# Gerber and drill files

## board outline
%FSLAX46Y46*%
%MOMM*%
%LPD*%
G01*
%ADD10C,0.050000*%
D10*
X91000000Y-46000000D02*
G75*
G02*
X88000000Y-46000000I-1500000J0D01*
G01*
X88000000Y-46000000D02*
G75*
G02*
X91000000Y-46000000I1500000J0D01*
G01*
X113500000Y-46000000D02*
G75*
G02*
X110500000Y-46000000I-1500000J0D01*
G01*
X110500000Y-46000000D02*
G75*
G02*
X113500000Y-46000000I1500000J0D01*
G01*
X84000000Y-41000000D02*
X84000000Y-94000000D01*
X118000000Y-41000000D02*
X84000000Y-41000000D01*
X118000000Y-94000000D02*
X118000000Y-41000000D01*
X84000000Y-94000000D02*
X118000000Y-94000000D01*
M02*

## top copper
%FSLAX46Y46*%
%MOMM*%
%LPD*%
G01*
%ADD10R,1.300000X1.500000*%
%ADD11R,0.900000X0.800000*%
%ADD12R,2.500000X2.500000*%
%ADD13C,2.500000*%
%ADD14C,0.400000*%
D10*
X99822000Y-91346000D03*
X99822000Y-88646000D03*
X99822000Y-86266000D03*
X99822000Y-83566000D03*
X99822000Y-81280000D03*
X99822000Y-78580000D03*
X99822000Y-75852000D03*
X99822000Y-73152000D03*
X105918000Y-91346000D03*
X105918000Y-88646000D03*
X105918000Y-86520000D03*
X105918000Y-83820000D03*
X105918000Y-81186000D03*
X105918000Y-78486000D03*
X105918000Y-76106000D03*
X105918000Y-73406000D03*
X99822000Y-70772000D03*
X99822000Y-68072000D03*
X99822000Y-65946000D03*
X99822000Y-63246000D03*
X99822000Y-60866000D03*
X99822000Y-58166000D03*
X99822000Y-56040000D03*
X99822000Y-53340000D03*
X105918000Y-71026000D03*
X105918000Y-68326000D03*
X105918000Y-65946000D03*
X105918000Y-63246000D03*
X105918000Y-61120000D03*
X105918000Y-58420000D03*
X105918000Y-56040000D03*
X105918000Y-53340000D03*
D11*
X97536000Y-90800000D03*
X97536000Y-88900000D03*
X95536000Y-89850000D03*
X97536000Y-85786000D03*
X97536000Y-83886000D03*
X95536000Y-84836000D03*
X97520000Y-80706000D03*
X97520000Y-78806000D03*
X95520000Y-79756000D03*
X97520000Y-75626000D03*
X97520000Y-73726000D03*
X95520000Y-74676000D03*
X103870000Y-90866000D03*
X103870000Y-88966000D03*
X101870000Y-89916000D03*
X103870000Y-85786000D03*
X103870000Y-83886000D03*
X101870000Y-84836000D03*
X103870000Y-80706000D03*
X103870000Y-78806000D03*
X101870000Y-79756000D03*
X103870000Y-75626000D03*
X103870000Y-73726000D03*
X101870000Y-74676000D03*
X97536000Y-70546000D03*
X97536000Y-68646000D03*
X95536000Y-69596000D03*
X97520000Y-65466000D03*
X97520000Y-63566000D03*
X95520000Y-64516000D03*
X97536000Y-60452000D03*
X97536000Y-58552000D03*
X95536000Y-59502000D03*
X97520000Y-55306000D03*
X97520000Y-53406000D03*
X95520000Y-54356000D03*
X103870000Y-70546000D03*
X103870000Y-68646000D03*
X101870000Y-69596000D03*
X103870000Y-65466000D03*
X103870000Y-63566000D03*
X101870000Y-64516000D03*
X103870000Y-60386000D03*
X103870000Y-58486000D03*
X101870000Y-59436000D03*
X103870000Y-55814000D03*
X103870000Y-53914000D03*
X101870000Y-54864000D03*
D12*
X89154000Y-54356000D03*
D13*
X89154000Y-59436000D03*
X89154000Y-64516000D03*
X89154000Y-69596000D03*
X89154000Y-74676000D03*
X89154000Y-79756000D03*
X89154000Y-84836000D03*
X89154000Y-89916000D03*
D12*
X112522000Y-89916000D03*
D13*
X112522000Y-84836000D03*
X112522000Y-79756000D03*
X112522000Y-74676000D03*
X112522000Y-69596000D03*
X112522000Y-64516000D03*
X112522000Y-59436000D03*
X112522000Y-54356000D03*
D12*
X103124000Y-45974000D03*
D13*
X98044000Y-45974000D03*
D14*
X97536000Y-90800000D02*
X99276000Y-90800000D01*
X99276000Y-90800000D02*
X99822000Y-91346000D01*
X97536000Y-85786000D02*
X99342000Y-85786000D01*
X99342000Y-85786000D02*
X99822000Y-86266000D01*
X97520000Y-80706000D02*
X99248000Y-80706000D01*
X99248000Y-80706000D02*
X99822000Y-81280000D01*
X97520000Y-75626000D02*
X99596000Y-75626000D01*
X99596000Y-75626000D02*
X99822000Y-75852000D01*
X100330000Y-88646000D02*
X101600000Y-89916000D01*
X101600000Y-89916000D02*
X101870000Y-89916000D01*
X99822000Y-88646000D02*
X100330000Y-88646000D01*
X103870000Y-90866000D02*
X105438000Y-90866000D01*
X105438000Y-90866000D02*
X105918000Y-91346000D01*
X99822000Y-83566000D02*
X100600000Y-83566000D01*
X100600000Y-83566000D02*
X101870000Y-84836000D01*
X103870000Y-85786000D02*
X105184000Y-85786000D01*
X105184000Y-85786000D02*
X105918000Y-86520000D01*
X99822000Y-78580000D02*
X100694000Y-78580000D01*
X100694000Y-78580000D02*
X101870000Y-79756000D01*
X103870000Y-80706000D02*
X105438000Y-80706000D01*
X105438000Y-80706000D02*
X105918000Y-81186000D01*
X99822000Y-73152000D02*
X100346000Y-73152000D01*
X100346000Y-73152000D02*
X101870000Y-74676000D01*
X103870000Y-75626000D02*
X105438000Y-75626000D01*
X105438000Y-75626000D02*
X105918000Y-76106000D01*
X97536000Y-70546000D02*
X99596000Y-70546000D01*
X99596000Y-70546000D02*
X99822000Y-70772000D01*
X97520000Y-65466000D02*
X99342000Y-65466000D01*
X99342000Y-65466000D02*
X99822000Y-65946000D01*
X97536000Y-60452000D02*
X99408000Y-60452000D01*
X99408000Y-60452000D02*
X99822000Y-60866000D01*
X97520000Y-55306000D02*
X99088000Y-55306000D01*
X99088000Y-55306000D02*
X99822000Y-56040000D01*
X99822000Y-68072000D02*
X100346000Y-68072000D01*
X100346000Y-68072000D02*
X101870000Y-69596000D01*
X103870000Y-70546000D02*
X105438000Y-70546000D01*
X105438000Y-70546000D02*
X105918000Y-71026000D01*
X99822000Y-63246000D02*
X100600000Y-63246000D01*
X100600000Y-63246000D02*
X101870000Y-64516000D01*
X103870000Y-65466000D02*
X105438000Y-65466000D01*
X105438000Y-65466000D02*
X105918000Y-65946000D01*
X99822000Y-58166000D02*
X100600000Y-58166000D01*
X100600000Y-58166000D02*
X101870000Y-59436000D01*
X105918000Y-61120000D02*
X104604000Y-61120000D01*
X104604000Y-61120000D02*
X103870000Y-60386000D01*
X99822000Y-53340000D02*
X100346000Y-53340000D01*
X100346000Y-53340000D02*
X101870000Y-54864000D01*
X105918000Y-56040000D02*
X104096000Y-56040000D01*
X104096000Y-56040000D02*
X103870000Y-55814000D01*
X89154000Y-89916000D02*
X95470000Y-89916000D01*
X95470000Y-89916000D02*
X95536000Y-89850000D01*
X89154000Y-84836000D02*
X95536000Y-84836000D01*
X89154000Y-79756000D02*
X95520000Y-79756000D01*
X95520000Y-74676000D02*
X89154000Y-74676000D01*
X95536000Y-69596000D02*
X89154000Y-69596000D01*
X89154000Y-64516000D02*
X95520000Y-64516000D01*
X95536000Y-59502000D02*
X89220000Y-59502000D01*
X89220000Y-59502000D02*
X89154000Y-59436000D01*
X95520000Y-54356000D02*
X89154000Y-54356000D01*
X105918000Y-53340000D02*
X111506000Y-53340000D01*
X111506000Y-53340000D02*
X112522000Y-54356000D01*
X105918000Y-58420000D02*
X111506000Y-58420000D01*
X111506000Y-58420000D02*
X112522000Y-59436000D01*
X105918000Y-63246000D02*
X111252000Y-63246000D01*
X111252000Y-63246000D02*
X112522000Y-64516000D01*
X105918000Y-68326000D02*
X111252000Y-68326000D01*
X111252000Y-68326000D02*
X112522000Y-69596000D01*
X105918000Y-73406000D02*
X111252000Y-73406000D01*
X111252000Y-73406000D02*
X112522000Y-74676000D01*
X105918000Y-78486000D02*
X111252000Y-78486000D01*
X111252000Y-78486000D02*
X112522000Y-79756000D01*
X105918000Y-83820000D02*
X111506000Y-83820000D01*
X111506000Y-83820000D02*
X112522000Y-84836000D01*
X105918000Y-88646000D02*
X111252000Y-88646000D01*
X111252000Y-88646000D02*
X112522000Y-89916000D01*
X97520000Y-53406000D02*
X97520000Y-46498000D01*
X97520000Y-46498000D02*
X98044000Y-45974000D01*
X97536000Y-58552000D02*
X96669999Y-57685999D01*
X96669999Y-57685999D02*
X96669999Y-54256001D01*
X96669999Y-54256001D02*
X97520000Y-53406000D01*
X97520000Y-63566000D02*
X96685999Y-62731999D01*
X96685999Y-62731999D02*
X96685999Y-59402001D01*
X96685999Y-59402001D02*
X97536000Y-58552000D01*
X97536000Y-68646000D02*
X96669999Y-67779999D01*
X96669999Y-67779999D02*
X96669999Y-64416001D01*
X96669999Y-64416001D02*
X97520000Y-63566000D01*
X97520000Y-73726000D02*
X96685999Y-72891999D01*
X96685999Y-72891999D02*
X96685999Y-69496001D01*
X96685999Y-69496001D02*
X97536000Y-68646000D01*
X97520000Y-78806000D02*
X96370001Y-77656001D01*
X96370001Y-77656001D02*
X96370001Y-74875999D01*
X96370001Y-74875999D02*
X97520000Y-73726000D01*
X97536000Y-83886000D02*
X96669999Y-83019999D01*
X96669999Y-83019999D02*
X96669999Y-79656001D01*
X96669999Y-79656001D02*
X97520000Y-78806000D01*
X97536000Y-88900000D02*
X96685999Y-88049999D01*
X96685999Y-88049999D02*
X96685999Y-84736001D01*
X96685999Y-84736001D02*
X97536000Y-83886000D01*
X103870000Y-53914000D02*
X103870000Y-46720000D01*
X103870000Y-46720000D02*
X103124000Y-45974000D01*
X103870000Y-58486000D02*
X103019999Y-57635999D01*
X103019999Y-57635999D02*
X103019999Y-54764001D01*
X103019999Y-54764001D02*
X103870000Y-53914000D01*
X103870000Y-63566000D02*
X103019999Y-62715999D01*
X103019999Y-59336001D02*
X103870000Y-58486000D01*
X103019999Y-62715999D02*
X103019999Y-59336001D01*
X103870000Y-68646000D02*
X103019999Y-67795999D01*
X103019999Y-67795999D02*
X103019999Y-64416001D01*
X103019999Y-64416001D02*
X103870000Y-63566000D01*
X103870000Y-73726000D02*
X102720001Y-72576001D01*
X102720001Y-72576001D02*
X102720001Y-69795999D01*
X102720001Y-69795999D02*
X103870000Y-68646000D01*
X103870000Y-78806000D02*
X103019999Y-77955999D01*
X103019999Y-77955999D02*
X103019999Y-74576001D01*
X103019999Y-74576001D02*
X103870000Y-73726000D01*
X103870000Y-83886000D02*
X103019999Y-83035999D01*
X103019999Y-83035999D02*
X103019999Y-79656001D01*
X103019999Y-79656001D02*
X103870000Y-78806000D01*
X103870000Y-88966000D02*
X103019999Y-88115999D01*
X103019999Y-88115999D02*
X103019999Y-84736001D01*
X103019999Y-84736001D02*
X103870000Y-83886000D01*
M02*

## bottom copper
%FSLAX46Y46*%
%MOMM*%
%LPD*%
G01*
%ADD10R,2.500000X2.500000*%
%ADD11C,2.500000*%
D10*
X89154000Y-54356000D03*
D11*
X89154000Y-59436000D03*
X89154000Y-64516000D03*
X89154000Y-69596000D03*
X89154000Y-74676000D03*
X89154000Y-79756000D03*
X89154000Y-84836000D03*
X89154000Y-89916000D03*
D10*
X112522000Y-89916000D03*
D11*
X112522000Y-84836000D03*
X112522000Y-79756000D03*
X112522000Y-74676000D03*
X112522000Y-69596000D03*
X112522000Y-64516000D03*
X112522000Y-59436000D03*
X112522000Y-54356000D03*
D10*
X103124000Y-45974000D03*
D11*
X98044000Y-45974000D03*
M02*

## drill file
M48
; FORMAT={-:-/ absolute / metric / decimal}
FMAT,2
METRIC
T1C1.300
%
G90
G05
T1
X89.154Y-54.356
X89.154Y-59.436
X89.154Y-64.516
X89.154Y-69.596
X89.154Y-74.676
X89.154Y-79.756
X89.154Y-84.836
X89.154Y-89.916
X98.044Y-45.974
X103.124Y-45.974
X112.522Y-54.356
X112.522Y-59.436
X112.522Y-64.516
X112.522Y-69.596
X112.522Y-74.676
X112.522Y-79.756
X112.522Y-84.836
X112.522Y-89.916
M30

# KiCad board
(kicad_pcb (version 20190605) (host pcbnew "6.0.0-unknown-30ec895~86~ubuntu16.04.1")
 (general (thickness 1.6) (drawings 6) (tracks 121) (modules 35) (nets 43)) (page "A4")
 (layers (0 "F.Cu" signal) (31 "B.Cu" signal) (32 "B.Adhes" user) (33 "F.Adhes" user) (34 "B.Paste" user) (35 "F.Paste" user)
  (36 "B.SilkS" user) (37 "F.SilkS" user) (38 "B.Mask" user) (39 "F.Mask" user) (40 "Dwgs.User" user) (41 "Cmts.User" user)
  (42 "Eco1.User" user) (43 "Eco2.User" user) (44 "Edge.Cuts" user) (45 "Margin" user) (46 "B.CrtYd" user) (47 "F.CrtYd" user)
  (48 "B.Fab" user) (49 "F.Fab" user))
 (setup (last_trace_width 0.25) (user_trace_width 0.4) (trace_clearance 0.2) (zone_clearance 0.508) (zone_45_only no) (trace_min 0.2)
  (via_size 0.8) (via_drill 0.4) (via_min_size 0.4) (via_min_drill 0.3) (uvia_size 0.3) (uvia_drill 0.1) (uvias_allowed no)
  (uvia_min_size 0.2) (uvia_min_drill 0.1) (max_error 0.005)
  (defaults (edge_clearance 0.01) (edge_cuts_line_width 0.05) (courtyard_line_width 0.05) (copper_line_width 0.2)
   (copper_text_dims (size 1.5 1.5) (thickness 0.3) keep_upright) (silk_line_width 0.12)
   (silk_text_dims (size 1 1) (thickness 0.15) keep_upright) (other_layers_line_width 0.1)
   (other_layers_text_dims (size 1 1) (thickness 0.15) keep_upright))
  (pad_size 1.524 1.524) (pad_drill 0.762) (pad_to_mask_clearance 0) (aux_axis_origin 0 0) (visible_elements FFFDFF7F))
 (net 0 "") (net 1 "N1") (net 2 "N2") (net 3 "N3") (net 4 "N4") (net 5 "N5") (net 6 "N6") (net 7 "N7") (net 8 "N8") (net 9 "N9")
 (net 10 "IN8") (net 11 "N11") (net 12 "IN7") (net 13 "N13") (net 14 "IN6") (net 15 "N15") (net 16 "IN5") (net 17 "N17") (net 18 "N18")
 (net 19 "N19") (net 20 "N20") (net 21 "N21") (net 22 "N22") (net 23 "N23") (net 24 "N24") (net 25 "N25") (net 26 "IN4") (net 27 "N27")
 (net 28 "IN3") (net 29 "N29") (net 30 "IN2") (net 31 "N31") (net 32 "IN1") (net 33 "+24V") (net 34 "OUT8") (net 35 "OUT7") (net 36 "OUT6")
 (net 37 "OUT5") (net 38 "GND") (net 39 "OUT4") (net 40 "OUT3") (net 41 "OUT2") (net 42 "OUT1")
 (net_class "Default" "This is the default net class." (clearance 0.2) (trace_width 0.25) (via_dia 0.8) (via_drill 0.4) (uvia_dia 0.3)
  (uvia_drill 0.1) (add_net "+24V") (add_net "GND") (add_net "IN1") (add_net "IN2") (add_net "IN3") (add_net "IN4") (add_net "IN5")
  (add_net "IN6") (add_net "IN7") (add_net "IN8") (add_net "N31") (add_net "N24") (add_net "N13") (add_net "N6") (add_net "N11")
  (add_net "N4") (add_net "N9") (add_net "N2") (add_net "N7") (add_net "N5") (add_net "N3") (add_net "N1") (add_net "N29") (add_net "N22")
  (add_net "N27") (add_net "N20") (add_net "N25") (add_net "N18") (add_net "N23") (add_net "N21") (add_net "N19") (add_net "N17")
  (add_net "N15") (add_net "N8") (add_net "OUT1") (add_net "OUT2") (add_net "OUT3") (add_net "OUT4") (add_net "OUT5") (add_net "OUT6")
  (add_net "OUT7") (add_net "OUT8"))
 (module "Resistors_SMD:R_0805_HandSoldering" (layer "F.Cu") (at 99.822 89.996 90)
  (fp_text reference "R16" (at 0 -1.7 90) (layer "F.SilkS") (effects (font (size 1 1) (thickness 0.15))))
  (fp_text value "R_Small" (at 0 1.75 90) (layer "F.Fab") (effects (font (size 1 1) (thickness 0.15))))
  (pad "1" smd rect (at -1.35 0 90) (size 1.5 1.3) (layers "F.Cu" "F.Paste" "F.Mask") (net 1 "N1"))
  (pad "2" smd rect (at 1.35 0 90) (size 1.5 1.3) (layers "F.Cu" "F.Paste" "F.Mask") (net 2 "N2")))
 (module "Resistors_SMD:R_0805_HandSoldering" (layer "F.Cu") (at 99.822 84.916 90)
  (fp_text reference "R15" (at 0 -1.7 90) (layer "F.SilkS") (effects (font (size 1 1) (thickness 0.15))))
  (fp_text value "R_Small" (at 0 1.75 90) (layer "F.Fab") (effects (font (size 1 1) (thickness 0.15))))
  (pad "1" smd rect (at -1.35 0 90) (size 1.5 1.3) (layers "F.Cu" "F.Paste" "F.Mask") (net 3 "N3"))
  (pad "2" smd rect (at 1.35 0 90) (size 1.5 1.3) (layers "F.Cu" "F.Paste" "F.Mask") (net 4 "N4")))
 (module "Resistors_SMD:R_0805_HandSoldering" (layer "F.Cu") (at 99.822 79.93 90)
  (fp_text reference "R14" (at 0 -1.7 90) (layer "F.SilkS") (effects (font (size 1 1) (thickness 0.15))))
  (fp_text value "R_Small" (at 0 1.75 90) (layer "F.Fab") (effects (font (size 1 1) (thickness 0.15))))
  (pad "1" smd rect (at -1.35 0 90) (size 1.5 1.3) (layers "F.Cu" "F.Paste" "F.Mask") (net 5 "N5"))
  (pad "2" smd rect (at 1.35 0 90) (size 1.5 1.3) (layers "F.Cu" "F.Paste" "F.Mask") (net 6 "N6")))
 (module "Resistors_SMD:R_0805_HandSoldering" (layer "F.Cu") (at 99.822 74.502 90)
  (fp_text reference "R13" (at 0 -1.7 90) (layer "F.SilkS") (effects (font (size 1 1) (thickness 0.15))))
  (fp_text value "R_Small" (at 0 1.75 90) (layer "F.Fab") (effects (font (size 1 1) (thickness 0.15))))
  (pad "1" smd rect (at -1.35 0 90) (size 1.5 1.3) (layers "F.Cu" "F.Paste" "F.Mask") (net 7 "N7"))
  (pad "2" smd rect (at 1.35 0 90) (size 1.5 1.3) (layers "F.Cu" "F.Paste" "F.Mask") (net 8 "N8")))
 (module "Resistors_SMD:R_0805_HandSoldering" (layer "F.Cu") (at 105.918 89.996 90)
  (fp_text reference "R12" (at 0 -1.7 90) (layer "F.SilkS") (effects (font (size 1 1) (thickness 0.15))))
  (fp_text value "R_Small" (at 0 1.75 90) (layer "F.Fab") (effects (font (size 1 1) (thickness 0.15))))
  (pad "1" smd rect (at -1.35 0 90) (size 1.5 1.3) (layers "F.Cu" "F.Paste" "F.Mask") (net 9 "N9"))
  (pad "2" smd rect (at 1.35 0 90) (size 1.5 1.3) (layers "F.Cu" "F.Paste" "F.Mask") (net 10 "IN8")))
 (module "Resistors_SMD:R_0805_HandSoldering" (layer "F.Cu") (at 105.918 85.17 90)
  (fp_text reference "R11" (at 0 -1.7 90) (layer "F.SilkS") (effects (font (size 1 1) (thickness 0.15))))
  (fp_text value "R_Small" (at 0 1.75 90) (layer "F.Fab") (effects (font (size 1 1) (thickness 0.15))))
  (pad "1" smd rect (at -1.35 0 90) (size 1.5 1.3) (layers "F.Cu" "F.Paste" "F.Mask") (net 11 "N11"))
  (pad "2" smd rect (at 1.35 0 90) (size 1.5 1.3) (layers "F.Cu" "F.Paste" "F.Mask") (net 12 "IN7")))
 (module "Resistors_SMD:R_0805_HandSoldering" (layer "F.Cu") (at 105.918 79.836 90)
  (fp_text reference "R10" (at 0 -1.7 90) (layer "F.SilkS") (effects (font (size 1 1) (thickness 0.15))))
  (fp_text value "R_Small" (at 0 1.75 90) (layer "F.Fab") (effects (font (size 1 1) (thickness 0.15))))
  (pad "1" smd rect (at -1.35 0 90) (size 1.5 1.3) (layers "F.Cu" "F.Paste" "F.Mask") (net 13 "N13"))
  (pad "2" smd rect (at 1.35 0 90) (size 1.5 1.3) (layers "F.Cu" "F.Paste" "F.Mask") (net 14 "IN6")))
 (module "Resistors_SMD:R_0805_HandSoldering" (layer "F.Cu") (at 105.918 74.756 90)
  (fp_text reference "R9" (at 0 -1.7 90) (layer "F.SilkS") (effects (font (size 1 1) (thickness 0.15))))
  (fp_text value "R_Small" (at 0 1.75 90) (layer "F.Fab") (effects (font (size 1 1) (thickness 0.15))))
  (pad "1" smd rect (at -1.35 0 90) (size 1.5 1.3) (layers "F.Cu" "F.Paste" "F.Mask") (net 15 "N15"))
  (pad "2" smd rect (at 1.35 0 90) (size 1.5 1.3) (layers "F.Cu" "F.Paste" "F.Mask") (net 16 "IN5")))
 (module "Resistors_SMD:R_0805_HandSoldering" (layer "F.Cu") (at 99.822 69.422 90)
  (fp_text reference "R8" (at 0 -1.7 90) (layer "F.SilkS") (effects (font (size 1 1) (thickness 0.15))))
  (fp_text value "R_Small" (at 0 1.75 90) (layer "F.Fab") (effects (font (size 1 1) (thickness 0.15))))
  (pad "1" smd rect (at -1.35 0 90) (size 1.5 1.3) (layers "F.Cu" "F.Paste" "F.Mask") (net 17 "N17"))
  (pad "2" smd rect (at 1.35 0 90) (size 1.5 1.3) (layers "F.Cu" "F.Paste" "F.Mask") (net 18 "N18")))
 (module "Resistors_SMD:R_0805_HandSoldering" (layer "F.Cu") (at 99.822 64.596 90)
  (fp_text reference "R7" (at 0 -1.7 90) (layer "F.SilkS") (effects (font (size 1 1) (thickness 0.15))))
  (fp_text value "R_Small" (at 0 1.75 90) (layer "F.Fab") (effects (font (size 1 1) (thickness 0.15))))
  (pad "1" smd rect (at -1.35 0 90) (size 1.5 1.3) (layers "F.Cu" "F.Paste" "F.Mask") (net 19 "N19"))
  (pad "2" smd rect (at 1.35 0 90) (size 1.5 1.3) (layers "F.Cu" "F.Paste" "F.Mask") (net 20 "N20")))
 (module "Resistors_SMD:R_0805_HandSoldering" (layer "F.Cu") (at 99.822 59.516 90)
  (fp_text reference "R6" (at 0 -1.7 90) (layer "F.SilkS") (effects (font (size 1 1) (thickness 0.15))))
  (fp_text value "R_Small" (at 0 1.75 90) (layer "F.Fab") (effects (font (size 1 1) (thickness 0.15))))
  (pad "1" smd rect (at -1.35 0 90) (size 1.5 1.3) (layers "F.Cu" "F.Paste" "F.Mask") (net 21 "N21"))
  (pad "2" smd rect (at 1.35 0 90) (size 1.5 1.3) (layers "F.Cu" "F.Paste" "F.Mask") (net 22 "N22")))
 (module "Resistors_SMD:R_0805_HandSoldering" (layer "F.Cu") (at 99.822 54.69 90)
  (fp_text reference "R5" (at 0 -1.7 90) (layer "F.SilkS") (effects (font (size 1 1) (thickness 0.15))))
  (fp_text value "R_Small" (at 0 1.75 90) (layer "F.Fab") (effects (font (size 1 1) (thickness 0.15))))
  (pad "1" smd rect (at -1.35 0 90) (size 1.5 1.3) (layers "F.Cu" "F.Paste" "F.Mask") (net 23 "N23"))
  (pad "2" smd rect (at 1.35 0 90) (size 1.5 1.3) (layers "F.Cu" "F.Paste" "F.Mask") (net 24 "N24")))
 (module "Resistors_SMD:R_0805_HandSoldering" (layer "F.Cu") (at 105.918 69.676 90)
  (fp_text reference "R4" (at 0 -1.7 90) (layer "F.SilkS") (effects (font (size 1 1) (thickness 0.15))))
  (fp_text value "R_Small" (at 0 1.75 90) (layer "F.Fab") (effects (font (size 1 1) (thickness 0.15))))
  (pad "1" smd rect (at -1.35 0 90) (size 1.5 1.3) (layers "F.Cu" "F.Paste" "F.Mask") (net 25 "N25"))
  (pad "2" smd rect (at 1.35 0 90) (size 1.5 1.3) (layers "F.Cu" "F.Paste" "F.Mask") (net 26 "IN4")))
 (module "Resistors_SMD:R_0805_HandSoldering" (layer "F.Cu") (at 105.918 64.596 90)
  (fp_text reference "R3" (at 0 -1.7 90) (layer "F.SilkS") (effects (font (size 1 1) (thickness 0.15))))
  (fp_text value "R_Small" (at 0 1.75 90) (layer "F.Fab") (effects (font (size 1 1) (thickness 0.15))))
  (pad "1" smd rect (at -1.35 0 90) (size 1.5 1.3) (layers "F.Cu" "F.Paste" "F.Mask") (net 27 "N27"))
  (pad "2" smd rect (at 1.35 0 90) (size 1.5 1.3) (layers "F.Cu" "F.Paste" "F.Mask") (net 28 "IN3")))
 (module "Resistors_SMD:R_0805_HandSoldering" (layer "F.Cu") (at 105.918 59.77 90)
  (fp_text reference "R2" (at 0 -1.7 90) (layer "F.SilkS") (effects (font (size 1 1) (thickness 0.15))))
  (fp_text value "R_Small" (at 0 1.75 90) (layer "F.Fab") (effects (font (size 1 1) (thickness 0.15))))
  (pad "1" smd rect (at -1.35 0 90) (size 1.5 1.3) (layers "F.Cu" "F.Paste" "F.Mask") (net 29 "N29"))
  (pad "2" smd rect (at 1.35 0 90) (size 1.5 1.3) (layers "F.Cu" "F.Paste" "F.Mask") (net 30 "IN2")))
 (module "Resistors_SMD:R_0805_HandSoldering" (layer "F.Cu") (at 105.918 54.69 90)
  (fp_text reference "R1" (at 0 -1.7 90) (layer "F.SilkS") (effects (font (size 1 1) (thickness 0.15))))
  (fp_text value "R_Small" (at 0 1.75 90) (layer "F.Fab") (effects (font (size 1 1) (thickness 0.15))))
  (pad "1" smd rect (at -1.35 0 90) (size 1.5 1.3) (layers "F.Cu" "F.Paste" "F.Mask") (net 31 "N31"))
  (pad "2" smd rect (at 1.35 0 90) (size 1.5 1.3) (layers "F.Cu" "F.Paste" "F.Mask") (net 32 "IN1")))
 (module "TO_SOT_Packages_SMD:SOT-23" (layer "F.Cu") (at 96.536 89.85 180)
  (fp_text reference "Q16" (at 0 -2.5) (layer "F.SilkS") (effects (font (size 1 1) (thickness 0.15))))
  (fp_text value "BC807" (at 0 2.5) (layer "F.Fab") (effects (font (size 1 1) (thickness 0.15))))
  (pad "1" smd rect (at -1 -0.95 180) (size 0.9 0.8) (layers "F.Cu" "F.Paste" "F.Mask") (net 1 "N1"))
  (pad "2" smd rect (at -1 0.95 180) (size 0.9 0.8) (layers "F.Cu" "F.Paste" "F.Mask") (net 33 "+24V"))
  (pad "3" smd rect (at 1 0 180) (size 0.9 0.8) (layers "F.Cu" "F.Paste" "F.Mask") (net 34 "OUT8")))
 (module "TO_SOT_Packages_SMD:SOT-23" (layer "F.Cu") (at 96.536 84.836 180)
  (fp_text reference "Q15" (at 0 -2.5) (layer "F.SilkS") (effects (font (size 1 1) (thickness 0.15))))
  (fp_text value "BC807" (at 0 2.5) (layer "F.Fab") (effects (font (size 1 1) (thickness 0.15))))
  (pad "1" smd rect (at -1 -0.95 180) (size 0.9 0.8) (layers "F.Cu" "F.Paste" "F.Mask") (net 3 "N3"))
  (pad "2" smd rect (at -1 0.95 180) (size 0.9 0.8) (layers "F.Cu" "F.Paste" "F.Mask") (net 33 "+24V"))
  (pad "3" smd rect (at 1 0 180) (size 0.9 0.8) (layers "F.Cu" "F.Paste" "F.Mask") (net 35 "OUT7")))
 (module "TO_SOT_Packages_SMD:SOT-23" (layer "F.Cu") (at 96.52 79.756 180)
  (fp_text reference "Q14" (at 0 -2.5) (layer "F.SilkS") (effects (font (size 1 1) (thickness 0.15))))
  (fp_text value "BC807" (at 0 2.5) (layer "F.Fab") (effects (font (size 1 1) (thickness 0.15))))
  (pad "1" smd rect (at -1 -0.95 180) (size 0.9 0.8) (layers "F.Cu" "F.Paste" "F.Mask") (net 5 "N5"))
  (pad "2" smd rect (at -1 0.95 180) (size 0.9 0.8) (layers "F.Cu" "F.Paste" "F.Mask") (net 33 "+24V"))
  (pad "3" smd rect (at 1 0 180) (size 0.9 0.8) (layers "F.Cu" "F.Paste" "F.Mask") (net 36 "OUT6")))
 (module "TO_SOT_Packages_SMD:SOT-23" (layer "F.Cu") (at 96.52 74.676 180)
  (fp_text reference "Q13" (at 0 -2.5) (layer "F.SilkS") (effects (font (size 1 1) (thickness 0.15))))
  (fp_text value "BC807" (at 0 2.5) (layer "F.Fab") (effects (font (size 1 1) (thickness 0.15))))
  (pad "1" smd rect (at -1 -0.95 180) (size 0.9 0.8) (layers "F.Cu" "F.Paste" "F.Mask") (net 7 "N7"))
  (pad "2" smd rect (at -1 0.95 180) (size 0.9 0.8) (layers "F.Cu" "F.Paste" "F.Mask") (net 33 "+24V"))
  (pad "3" smd rect (at 1 0 180) (size 0.9 0.8) (layers "F.Cu" "F.Paste" "F.Mask") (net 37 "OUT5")))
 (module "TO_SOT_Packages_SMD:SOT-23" (layer "F.Cu") (at 102.87 89.916 180)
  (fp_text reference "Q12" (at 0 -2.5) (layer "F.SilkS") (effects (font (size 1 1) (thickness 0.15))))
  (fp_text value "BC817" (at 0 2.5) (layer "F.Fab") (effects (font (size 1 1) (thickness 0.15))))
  (pad "1" smd rect (at -1 -0.95 180) (size 0.9 0.8) (layers "F.Cu" "F.Paste" "F.Mask") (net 9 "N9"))
  (pad "2" smd rect (at -1 0.95 180) (size 0.9 0.8) (layers "F.Cu" "F.Paste" "F.Mask") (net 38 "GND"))
  (pad "3" smd rect (at 1 0 180) (size 0.9 0.8) (layers "F.Cu" "F.Paste" "F.Mask") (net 2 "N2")))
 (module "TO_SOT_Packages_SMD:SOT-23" (layer "F.Cu") (at 102.87 84.836 180)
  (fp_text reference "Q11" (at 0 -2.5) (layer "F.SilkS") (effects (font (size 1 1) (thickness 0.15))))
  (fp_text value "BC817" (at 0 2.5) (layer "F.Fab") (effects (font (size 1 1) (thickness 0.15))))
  (pad "1" smd rect (at -1 -0.95 180) (size 0.9 0.8) (layers "F.Cu" "F.Paste" "F.Mask") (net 11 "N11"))
  (pad "2" smd rect (at -1 0.95 180) (size 0.9 0.8) (layers "F.Cu" "F.Paste" "F.Mask") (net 38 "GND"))
  (pad "3" smd rect (at 1 0 180) (size 0.9 0.8) (layers "F.Cu" "F.Paste" "F.Mask") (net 4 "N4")))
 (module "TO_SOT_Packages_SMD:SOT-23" (layer "F.Cu") (at 102.87 79.756 180)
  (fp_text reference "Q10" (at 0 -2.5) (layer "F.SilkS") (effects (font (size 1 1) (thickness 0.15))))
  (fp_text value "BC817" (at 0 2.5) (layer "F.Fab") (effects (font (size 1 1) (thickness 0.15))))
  (pad "1" smd rect (at -1 -0.95 180) (size 0.9 0.8) (layers "F.Cu" "F.Paste" "F.Mask") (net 13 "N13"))
  (pad "2" smd rect (at -1 0.95 180) (size 0.9 0.8) (layers "F.Cu" "F.Paste" "F.Mask") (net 38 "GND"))
  (pad "3" smd rect (at 1 0 180) (size 0.9 0.8) (layers "F.Cu" "F.Paste" "F.Mask") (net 6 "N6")))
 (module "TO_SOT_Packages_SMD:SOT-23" (layer "F.Cu") (at 102.87 74.676 180)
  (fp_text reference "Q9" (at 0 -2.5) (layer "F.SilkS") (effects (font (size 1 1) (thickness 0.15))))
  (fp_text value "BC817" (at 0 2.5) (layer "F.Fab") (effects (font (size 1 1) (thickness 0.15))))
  (pad "1" smd rect (at -1 -0.95 180) (size 0.9 0.8) (layers "F.Cu" "F.Paste" "F.Mask") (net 15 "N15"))
  (pad "2" smd rect (at -1 0.95 180) (size 0.9 0.8) (layers "F.Cu" "F.Paste" "F.Mask") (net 38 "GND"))
  (pad "3" smd rect (at 1 0 180) (size 0.9 0.8) (layers "F.Cu" "F.Paste" "F.Mask") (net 8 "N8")))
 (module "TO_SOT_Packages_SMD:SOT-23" (layer "F.Cu") (at 96.536 69.596 180)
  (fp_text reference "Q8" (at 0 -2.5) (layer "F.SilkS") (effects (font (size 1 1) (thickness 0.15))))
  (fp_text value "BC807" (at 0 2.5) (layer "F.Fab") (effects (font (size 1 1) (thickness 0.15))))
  (pad "1" smd rect (at -1 -0.95 180) (size 0.9 0.8) (layers "F.Cu" "F.Paste" "F.Mask") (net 17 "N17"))
  (pad "2" smd rect (at -1 0.95 180) (size 0.9 0.8) (layers "F.Cu" "F.Paste" "F.Mask") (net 33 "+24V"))
  (pad "3" smd rect (at 1 0 180) (size 0.9 0.8) (layers "F.Cu" "F.Paste" "F.Mask") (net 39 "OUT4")))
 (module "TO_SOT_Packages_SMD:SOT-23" (layer "F.Cu") (at 96.52 64.516 180)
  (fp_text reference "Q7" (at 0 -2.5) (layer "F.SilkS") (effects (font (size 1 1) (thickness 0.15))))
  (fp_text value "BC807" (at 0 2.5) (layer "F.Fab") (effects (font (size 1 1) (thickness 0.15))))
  (pad "1" smd rect (at -1 -0.95 180) (size 0.9 0.8) (layers "F.Cu" "F.Paste" "F.Mask") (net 19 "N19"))
  (pad "2" smd rect (at -1 0.95 180) (size 0.9 0.8) (layers "F.Cu" "F.Paste" "F.Mask") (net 33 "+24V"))
  (pad "3" smd rect (at 1 0 180) (size 0.9 0.8) (layers "F.Cu" "F.Paste" "F.Mask") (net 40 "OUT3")))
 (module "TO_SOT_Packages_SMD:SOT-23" (layer "F.Cu") (at 96.536 59.502 180)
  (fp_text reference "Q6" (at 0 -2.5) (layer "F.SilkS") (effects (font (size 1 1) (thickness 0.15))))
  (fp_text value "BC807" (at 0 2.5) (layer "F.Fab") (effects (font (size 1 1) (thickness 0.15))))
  (pad "1" smd rect (at -1 -0.95 180) (size 0.9 0.8) (layers "F.Cu" "F.Paste" "F.Mask") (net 21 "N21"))
  (pad "2" smd rect (at -1 0.95 180) (size 0.9 0.8) (layers "F.Cu" "F.Paste" "F.Mask") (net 33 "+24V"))
  (pad "3" smd rect (at 1 0 180) (size 0.9 0.8) (layers "F.Cu" "F.Paste" "F.Mask") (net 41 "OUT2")))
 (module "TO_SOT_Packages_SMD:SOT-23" (layer "F.Cu") (at 96.52 54.356 180)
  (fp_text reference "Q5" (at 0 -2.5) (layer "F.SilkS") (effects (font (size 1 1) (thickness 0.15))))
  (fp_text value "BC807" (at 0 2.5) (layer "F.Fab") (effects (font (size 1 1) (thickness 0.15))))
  (pad "1" smd rect (at -1 -0.95 180) (size 0.9 0.8) (layers "F.Cu" "F.Paste" "F.Mask") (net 23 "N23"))
  (pad "2" smd rect (at -1 0.95 180) (size 0.9 0.8) (layers "F.Cu" "F.Paste" "F.Mask") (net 33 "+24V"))
  (pad "3" smd rect (at 1 0 180) (size 0.9 0.8) (layers "F.Cu" "F.Paste" "F.Mask") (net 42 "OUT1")))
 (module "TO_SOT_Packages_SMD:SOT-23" (layer "F.Cu") (at 102.87 69.596 180)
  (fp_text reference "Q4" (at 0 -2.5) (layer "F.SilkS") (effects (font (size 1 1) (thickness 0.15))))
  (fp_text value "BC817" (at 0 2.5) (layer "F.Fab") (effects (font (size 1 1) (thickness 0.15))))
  (pad "1" smd rect (at -1 -0.95 180) (size 0.9 0.8) (layers "F.Cu" "F.Paste" "F.Mask") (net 25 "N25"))
  (pad "2" smd rect (at -1 0.95 180) (size 0.9 0.8) (layers "F.Cu" "F.Paste" "F.Mask") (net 38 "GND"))
  (pad "3" smd rect (at 1 0 180) (size 0.9 0.8) (layers "F.Cu" "F.Paste" "F.Mask") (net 18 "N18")))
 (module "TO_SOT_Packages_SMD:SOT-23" (layer "F.Cu") (at 102.87 64.516 180)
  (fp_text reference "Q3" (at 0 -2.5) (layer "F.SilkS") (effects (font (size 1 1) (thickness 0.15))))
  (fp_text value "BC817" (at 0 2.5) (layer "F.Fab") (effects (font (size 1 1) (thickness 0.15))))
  (pad "1" smd rect (at -1 -0.95 180) (size 0.9 0.8) (layers "F.Cu" "F.Paste" "F.Mask") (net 27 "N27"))
  (pad "2" smd rect (at -1 0.95 180) (size 0.9 0.8) (layers "F.Cu" "F.Paste" "F.Mask") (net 38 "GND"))
  (pad "3" smd rect (at 1 0 180) (size 0.9 0.8) (layers "F.Cu" "F.Paste" "F.Mask") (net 20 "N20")))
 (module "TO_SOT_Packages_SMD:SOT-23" (layer "F.Cu") (at 102.87 59.436 180)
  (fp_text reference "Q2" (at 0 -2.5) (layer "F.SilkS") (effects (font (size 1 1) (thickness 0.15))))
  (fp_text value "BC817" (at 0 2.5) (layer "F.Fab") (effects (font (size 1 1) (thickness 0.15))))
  (pad "1" smd rect (at -1 -0.95 180) (size 0.9 0.8) (layers "F.Cu" "F.Paste" "F.Mask") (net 29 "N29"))
  (pad "2" smd rect (at -1 0.95 180) (size 0.9 0.8) (layers "F.Cu" "F.Paste" "F.Mask") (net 38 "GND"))
  (pad "3" smd rect (at 1 0 180) (size 0.9 0.8) (layers "F.Cu" "F.Paste" "F.Mask") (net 22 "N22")))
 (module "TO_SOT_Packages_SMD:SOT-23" (layer "F.Cu") (at 102.87 54.864 180)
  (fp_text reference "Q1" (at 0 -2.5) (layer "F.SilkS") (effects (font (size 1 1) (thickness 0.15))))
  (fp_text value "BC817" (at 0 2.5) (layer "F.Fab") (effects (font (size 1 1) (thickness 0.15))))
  (pad "1" smd rect (at -1 -0.95 180) (size 0.9 0.8) (layers "F.Cu" "F.Paste" "F.Mask") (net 31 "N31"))
  (pad "2" smd rect (at -1 0.95 180) (size 0.9 0.8) (layers "F.Cu" "F.Paste" "F.Mask") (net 38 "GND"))
  (pad "3" smd rect (at 1 0 180) (size 0.9 0.8) (layers "F.Cu" "F.Paste" "F.Mask") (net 24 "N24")))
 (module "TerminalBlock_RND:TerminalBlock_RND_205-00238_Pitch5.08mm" (layer "F.Cu") (at 89.154 54.356 270)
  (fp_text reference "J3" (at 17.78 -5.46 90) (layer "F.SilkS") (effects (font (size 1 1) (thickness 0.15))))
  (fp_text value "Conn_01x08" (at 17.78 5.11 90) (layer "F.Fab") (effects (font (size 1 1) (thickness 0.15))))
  (pad "1" thru_hole rect (at 0 0 270) (size 2.5 2.5) (drill 1.3) (layers *.Cu *.Mask) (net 42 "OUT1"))
  (pad "2" thru_hole circle (at 5.08 0 270) (size 2.5 2.5) (drill 1.3) (layers *.Cu *.Mask) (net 41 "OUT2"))
  (pad "3" thru_hole circle (at 10.16 0 270) (size 2.5 2.5) (drill 1.3) (layers *.Cu *.Mask) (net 40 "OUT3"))
  (pad "4" thru_hole circle (at 15.24 0 270) (size 2.5 2.5) (drill 1.3) (layers *.Cu *.Mask) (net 39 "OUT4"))
  (pad "5" thru_hole circle (at 20.32 0 270) (size 2.5 2.5) (drill 1.3) (layers *.Cu *.Mask) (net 37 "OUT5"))
  (pad "6" thru_hole circle (at 25.4 0 270) (size 2.5 2.5) (drill 1.3) (layers *.Cu *.Mask) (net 36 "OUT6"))
  (pad "7" thru_hole circle (at 30.48 0 270) (size 2.5 2.5) (drill 1.3) (layers *.Cu *.Mask) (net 35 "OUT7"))
  (pad "8" thru_hole circle (at 35.56 0 270) (size 2.5 2.5) (drill 1.3) (layers *.Cu *.Mask) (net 34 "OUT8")))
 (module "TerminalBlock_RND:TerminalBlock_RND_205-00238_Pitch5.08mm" (layer "F.Cu") (at 112.522 89.916 90)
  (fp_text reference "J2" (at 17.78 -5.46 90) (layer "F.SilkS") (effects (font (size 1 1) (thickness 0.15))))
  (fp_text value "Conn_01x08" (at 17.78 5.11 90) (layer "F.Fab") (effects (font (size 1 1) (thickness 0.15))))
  (pad "1" thru_hole rect (at 0 0 90) (size 2.5 2.5) (drill 1.3) (layers *.Cu *.Mask) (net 10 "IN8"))
  (pad "2" thru_hole circle (at 5.08 0 90) (size 2.5 2.5) (drill 1.3) (layers *.Cu *.Mask) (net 12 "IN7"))
  (pad "3" thru_hole circle (at 10.16 0 90) (size 2.5 2.5) (drill 1.3) (layers *.Cu *.Mask) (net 14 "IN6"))
  (pad "4" thru_hole circle (at 15.24 0 90) (size 2.5 2.5) (drill 1.3) (layers *.Cu *.Mask) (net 16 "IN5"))
  (pad "5" thru_hole circle (at 20.32 0 90) (size 2.5 2.5) (drill 1.3) (layers *.Cu *.Mask) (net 26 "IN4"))
  (pad "6" thru_hole circle (at 25.4 0 90) (size 2.5 2.5) (drill 1.3) (layers *.Cu *.Mask) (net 28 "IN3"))
  (pad "7" thru_hole circle (at 30.48 0 90) (size 2.5 2.5) (drill 1.3) (layers *.Cu *.Mask) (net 30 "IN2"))
  (pad "8" thru_hole circle (at 35.56 0 90) (size 2.5 2.5) (drill 1.3) (layers *.Cu *.Mask) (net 32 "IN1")))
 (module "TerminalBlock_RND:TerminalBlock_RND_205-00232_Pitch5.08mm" (layer "F.Cu") (at 103.124 45.974 180)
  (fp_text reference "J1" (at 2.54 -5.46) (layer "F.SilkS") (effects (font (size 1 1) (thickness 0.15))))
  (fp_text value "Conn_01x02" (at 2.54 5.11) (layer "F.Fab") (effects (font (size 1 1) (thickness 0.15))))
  (pad "1" thru_hole rect (at 0 0 180) (size 2.5 2.5) (drill 1.3) (layers *.Cu *.Mask) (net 38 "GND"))
  (pad "2" thru_hole circle (at 5.08 0 180) (size 2.5 2.5) (drill 1.3) (layers *.Cu *.Mask) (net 33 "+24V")))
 (gr_circle (center 89.5 46) (end 91 46) (layer "Edge.Cuts") (width 0.05))
 (gr_circle (center 112 46) (end 113.5 46) (layer "Edge.Cuts") (width 0.05))
 (gr_line (start 84 41) (end 84 94) (layer "Edge.Cuts") (width 0.05))
 (gr_line (start 118 41) (end 84 41) (layer "Edge.Cuts") (width 0.05))
 (gr_line (start 118 94) (end 118 41) (layer "Edge.Cuts") (width 0.05))
 (gr_line (start 84 94) (end 118 94) (layer "Edge.Cuts") (width 0.05))
 (segment (start 97.536 90.8) (end 99.276 90.8) (width 0.4) (layer "F.Cu") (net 1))
 (segment (start 99.276 90.8) (end 99.822 91.346) (width 0.4) (layer "F.Cu") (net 1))
 (segment (start 97.536 85.786) (end 99.342 85.786) (width 0.4) (layer "F.Cu") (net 3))
 (segment (start 99.342 85.786) (end 99.822 86.266) (width 0.4) (layer "F.Cu") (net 3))
 (segment (start 97.52 80.706) (end 99.248 80.706) (width 0.4) (layer "F.Cu") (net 5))
 (segment (start 99.248 80.706) (end 99.822 81.28) (width 0.4) (layer "F.Cu") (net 5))
 (segment (start 97.52 75.626) (end 99.596 75.626) (width 0.4) (layer "F.Cu") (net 7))
 (segment (start 99.596 75.626) (end 99.822 75.852) (width 0.4) (layer "F.Cu") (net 7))
 (segment (start 100.33 88.646) (end 101.6 89.916) (width 0.4) (layer "F.Cu") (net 2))
 (segment (start 101.6 89.916) (end 101.87 89.916) (width 0.4) (layer "F.Cu") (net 2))
 (segment (start 99.822 88.646) (end 100.33 88.646) (width 0.4) (layer "F.Cu") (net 2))
 (segment (start 103.87 90.866) (end 105.438 90.866) (width 0.4) (layer "F.Cu") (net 9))
 (segment (start 105.438 90.866) (end 105.918 91.346) (width 0.4) (layer "F.Cu") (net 9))
 (segment (start 99.822 83.566) (end 100.6 83.566) (width 0.4) (layer "F.Cu") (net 4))
 (segment (start 100.6 83.566) (end 101.87 84.836) (width 0.4) (layer "F.Cu") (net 4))
 (segment (start 103.87 85.786) (end 105.184 85.786) (width 0.4) (layer "F.Cu") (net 11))
 (segment (start 105.184 85.786) (end 105.918 86.52) (width 0.4) (layer "F.Cu") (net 11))
 (segment (start 99.822 78.58) (end 100.694 78.58) (width 0.4) (layer "F.Cu") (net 6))
 (segment (start 100.694 78.58) (end 101.87 79.756) (width 0.4) (layer "F.Cu") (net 6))
 (segment (start 103.87 80.706) (end 105.438 80.706) (width 0.4) (layer "F.Cu") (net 13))
 (segment (start 105.438 80.706) (end 105.918 81.186) (width 0.4) (layer "F.Cu") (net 13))
 (segment (start 99.822 73.152) (end 100.346 73.152) (width 0.4) (layer "F.Cu") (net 8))
 (segment (start 100.346 73.152) (end 101.87 74.676) (width 0.4) (layer "F.Cu") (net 8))
 (segment (start 103.87 75.626) (end 105.438 75.626) (width 0.4) (layer "F.Cu") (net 15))
 (segment (start 105.438 75.626) (end 105.918 76.106) (width 0.4) (layer "F.Cu") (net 15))
 (segment (start 97.536 70.546) (end 99.596 70.546) (width 0.4) (layer "F.Cu") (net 17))
 (segment (start 99.596 70.546) (end 99.822 70.772) (width 0.4) (layer "F.Cu") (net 17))
 (segment (start 97.52 65.466) (end 99.342 65.466) (width 0.4) (layer "F.Cu") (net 19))
 (segment (start 99.342 65.466) (end 99.822 65.946) (width 0.4) (layer "F.Cu") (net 19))
 (segment (start 97.536 60.452) (end 99.408 60.452) (width 0.4) (layer "F.Cu") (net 21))
 (segment (start 99.408 60.452) (end 99.822 60.866) (width 0.4) (layer "F.Cu") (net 21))
 (segment (start 97.52 55.306) (end 99.088 55.306) (width 0.4) (layer "F.Cu") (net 23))
 (segment (start 99.088 55.306) (end 99.822 56.04) (width 0.4) (layer "F.Cu") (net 23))
 (segment (start 99.822 68.072) (end 100.346 68.072) (width 0.4) (layer "F.Cu") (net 18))
 (segment (start 100.346 68.072) (end 101.87 69.596) (width 0.4) (layer "F.Cu") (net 18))
 (segment (start 103.87 70.546) (end 105.438 70.546) (width 0.4) (layer "F.Cu") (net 25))
 (segment (start 105.438 70.546) (end 105.918 71.026) (width 0.4) (layer "F.Cu") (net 25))
 (segment (start 99.822 63.246) (end 100.6 63.246) (width 0.4) (layer "F.Cu") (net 20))
 (segment (start 100.6 63.246) (end 101.87 64.516) (width 0.4) (layer "F.Cu") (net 20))
 (segment (start 103.87 65.466) (end 105.438 65.466) (width 0.4) (layer "F.Cu") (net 27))
 (segment (start 105.438 65.466) (end 105.918 65.946) (width 0.4) (layer "F.Cu") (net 27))
 (segment (start 99.822 58.166) (end 100.6 58.166) (width 0.4) (layer "F.Cu") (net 22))
 (segment (start 100.6 58.166) (end 101.87 59.436) (width 0.4) (layer "F.Cu") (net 22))
 (segment (start 105.918 61.12) (end 104.604 61.12) (width 0.4) (layer "F.Cu") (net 29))
 (segment (start 104.604 61.12) (end 103.87 60.386) (width 0.4) (layer "F.Cu") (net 29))
 (segment (start 99.822 53.34) (end 100.346 53.34) (width 0.4) (layer "F.Cu") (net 24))
 (segment (start 100.346 53.34) (end 101.87 54.864) (width 0.4) (layer "F.Cu") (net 24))
 (segment (start 105.918 56.04) (end 104.096 56.04) (width 0.4) (layer "F.Cu") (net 31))
 (segment (start 104.096 56.04) (end 103.87 55.814) (width 0.4) (layer "F.Cu") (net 31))
 (segment (start 89.154 89.916) (end 95.47 89.916) (width 0.4) (layer "F.Cu") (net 34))
 (segment (start 95.47 89.916) (end 95.536 89.85) (width 0.4) (layer "F.Cu") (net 34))
 (segment (start 89.154 84.836) (end 95.536 84.836) (width 0.4) (layer "F.Cu") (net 35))
 (segment (start 89.154 79.756) (end 95.52 79.756) (width 0.4) (layer "F.Cu") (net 36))
 (segment (start 95.52 74.676) (end 89.154 74.676) (width 0.4) (layer "F.Cu") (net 37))
 (segment (start 95.536 69.596) (end 89.154 69.596) (width 0.4) (layer "F.Cu") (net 39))
 (segment (start 89.154 64.516) (end 95.52 64.516) (width 0.4) (layer "F.Cu") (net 40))
 (segment (start 95.536 59.502) (end 89.22 59.502) (width 0.4) (layer "F.Cu") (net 41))
 (segment (start 89.22 59.502) (end 89.154 59.436) (width 0.4) (layer "F.Cu") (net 41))
 (segment (start 95.52 54.356) (end 89.154 54.356) (width 0.4) (layer "F.Cu") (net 42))
 (segment (start 105.918 53.34) (end 111.506 53.34) (width 0.4) (layer "F.Cu") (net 32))
 (segment (start 111.506 53.34) (end 112.522 54.356) (width 0.4) (layer "F.Cu") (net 32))
 (segment (start 105.918 58.42) (end 111.506 58.42) (width 0.4) (layer "F.Cu") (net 30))
 (segment (start 111.506 58.42) (end 112.522 59.436) (width 0.4) (layer "F.Cu") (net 30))
 (segment (start 105.918 63.246) (end 111.252 63.246) (width 0.4) (layer "F.Cu") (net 28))
 (segment (start 111.252 63.246) (end 112.522 64.516) (width 0.4) (layer "F.Cu") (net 28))
 (segment (start 105.918 68.326) (end 111.252 68.326) (width 0.4) (layer "F.Cu") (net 26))
 (segment (start 111.252 68.326) (end 112.522 69.596) (width 0.4) (layer "F.Cu") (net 26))
 (segment (start 105.918 73.406) (end 111.252 73.406) (width 0.4) (layer "F.Cu") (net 16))
 (segment (start 111.252 73.406) (end 112.522 74.676) (width 0.4) (layer "F.Cu") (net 16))
 (segment (start 105.918 78.486) (end 111.252 78.486) (width 0.4) (layer "F.Cu") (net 14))
 (segment (start 111.252 78.486) (end 112.522 79.756) (width 0.4) (layer "F.Cu") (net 14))
 (segment (start 105.918 83.82) (end 111.506 83.82) (width 0.4) (layer "F.Cu") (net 12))
 (segment (start 111.506 83.82) (end 112.522 84.836) (width 0.4) (layer "F.Cu") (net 12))
 (segment (start 105.918 88.646) (end 111.252 88.646) (width 0.4) (layer "F.Cu") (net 10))
 (segment (start 111.252 88.646) (end 112.522 89.916) (width 0.4) (layer "F.Cu") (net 10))
 (segment (start 97.52 53.406) (end 97.52 46.498) (width 0.4) (layer "F.Cu") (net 33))
 (segment (start 97.52 46.498) (end 98.044 45.974) (width 0.4) (layer "F.Cu") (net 33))
 (segment (start 97.536 58.552) (end 96.669999 57.685999) (width 0.4) (layer "F.Cu") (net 33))
 (segment (start 96.669999 57.685999) (end 96.669999 54.256001) (width 0.4) (layer "F.Cu") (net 33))
 (segment (start 96.669999 54.256001) (end 97.52 53.406) (width 0.4) (layer "F.Cu") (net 33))
 (segment (start 97.52 63.566) (end 96.685999 62.731999) (width 0.4) (layer "F.Cu") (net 33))
 (segment (start 96.685999 62.731999) (end 96.685999 59.402001) (width 0.4) (layer "F.Cu") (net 33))
 (segment (start 96.685999 59.402001) (end 97.536 58.552) (width 0.4) (layer "F.Cu") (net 33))
 (segment (start 97.536 68.646) (end 96.669999 67.779999) (width 0.4) (layer "F.Cu") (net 33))
 (segment (start 96.669999 67.779999) (end 96.669999 64.416001) (width 0.4) (layer "F.Cu") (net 33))
 (segment (start 96.669999 64.416001) (end 97.52 63.566) (width 0.4) (layer "F.Cu") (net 33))
 (segment (start 97.52 73.726) (end 96.685999 72.891999) (width 0.4) (layer "F.Cu") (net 33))
 (segment (start 96.685999 72.891999) (end 96.685999 69.496001) (width 0.4) (layer "F.Cu") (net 33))
 (segment (start 96.685999 69.496001) (end 97.536 68.646) (width 0.4) (layer "F.Cu") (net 33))
 (segment (start 97.52 78.806) (end 96.370001 77.656001) (width 0.4) (layer "F.Cu") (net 33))
 (segment (start 96.370001 77.656001) (end 96.370001 74.875999) (width 0.4) (layer "F.Cu") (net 33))
 (segment (start 96.370001 74.875999) (end 97.52 73.726) (width 0.4) (layer "F.Cu") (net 33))
 (segment (start 97.536 83.886) (end 96.669999 83.019999) (width 0.4) (layer "F.Cu") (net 33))
 (segment (start 96.669999 83.019999) (end 96.669999 79.656001) (width 0.4) (layer "F.Cu") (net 33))
 (segment (start 96.669999 79.656001) (end 97.52 78.806) (width 0.4) (layer "F.Cu") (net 33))
 (segment (start 97.536 88.9) (end 96.685999 88.049999) (width 0.4) (layer "F.Cu") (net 33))
 (segment (start 96.685999 88.049999) (end 96.685999 84.736001) (width 0.4) (layer "F.Cu") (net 33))
 (segment (start 96.685999 84.736001) (end 97.536 83.886) (width 0.4) (layer "F.Cu") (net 33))
 (segment (start 103.87 53.914) (end 103.87 46.72) (width 0.4) (layer "F.Cu") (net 38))
 (segment (start 103.87 46.72) (end 103.124 45.974) (width 0.4) (layer "F.Cu") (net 38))
 (segment (start 103.87 58.486) (end 103.019999 57.635999) (width 0.4) (layer "F.Cu") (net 38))
 (segment (start 103.019999 57.635999) (end 103.019999 54.764001) (width 0.4) (layer "F.Cu") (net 38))
 (segment (start 103.019999 54.764001) (end 103.87 53.914) (width 0.4) (layer "F.Cu") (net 38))
 (segment (start 103.87 63.566) (end 103.019999 62.715999) (width 0.4) (layer "F.Cu") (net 38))
 (segment (start 103.019999 59.336001) (end 103.87 58.486) (width 0.4) (layer "F.Cu") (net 38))
 (segment (start 103.019999 62.715999) (end 103.019999 59.336001) (width 0.4) (layer "F.Cu") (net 38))
 (segment (start 103.87 68.646) (end 103.019999 67.795999) (width 0.4) (layer "F.Cu") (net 38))
 (segment (start 103.019999 67.795999) (end 103.019999 64.416001) (width 0.4) (layer "F.Cu") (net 38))
 (segment (start 103.019999 64.416001) (end 103.87 63.566) (width 0.4) (layer "F.Cu") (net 38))
 (segment (start 103.87 73.726) (end 102.720001 72.576001) (width 0.4) (layer "F.Cu") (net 38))
 (segment (start 102.720001 72.576001) (end 102.720001 69.795999) (width 0.4) (layer "F.Cu") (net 38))
 (segment (start 102.720001 69.795999) (end 103.87 68.646) (width 0.4) (layer "F.Cu") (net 38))
 (segment (start 103.87 78.806) (end 103.019999 77.955999) (width 0.4) (layer "F.Cu") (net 38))
 (segment (start 103.019999 77.955999) (end 103.019999 74.576001) (width 0.4) (layer "F.Cu") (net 38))
 (segment (start 103.019999 74.576001) (end 103.87 73.726) (width 0.4) (layer "F.Cu") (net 38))
 (segment (start 103.87 83.886) (end 103.019999 83.035999) (width 0.4) (layer "F.Cu") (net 38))
 (segment (start 103.019999 83.035999) (end 103.019999 79.656001) (width 0.4) (layer "F.Cu") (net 38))
 (segment (start 103.019999 79.656001) (end 103.87 78.806) (width 0.4) (layer "F.Cu") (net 38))
 (segment (start 103.87 88.966) (end 103.019999 88.115999) (width 0.4) (layer "F.Cu") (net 38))
 (segment (start 103.019999 88.115999) (end 103.019999 84.736001) (width 0.4) (layer "F.Cu") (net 38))
 (segment (start 103.019999 84.736001) (end 103.87 83.886) (width 0.4) (layer "F.Cu") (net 38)))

